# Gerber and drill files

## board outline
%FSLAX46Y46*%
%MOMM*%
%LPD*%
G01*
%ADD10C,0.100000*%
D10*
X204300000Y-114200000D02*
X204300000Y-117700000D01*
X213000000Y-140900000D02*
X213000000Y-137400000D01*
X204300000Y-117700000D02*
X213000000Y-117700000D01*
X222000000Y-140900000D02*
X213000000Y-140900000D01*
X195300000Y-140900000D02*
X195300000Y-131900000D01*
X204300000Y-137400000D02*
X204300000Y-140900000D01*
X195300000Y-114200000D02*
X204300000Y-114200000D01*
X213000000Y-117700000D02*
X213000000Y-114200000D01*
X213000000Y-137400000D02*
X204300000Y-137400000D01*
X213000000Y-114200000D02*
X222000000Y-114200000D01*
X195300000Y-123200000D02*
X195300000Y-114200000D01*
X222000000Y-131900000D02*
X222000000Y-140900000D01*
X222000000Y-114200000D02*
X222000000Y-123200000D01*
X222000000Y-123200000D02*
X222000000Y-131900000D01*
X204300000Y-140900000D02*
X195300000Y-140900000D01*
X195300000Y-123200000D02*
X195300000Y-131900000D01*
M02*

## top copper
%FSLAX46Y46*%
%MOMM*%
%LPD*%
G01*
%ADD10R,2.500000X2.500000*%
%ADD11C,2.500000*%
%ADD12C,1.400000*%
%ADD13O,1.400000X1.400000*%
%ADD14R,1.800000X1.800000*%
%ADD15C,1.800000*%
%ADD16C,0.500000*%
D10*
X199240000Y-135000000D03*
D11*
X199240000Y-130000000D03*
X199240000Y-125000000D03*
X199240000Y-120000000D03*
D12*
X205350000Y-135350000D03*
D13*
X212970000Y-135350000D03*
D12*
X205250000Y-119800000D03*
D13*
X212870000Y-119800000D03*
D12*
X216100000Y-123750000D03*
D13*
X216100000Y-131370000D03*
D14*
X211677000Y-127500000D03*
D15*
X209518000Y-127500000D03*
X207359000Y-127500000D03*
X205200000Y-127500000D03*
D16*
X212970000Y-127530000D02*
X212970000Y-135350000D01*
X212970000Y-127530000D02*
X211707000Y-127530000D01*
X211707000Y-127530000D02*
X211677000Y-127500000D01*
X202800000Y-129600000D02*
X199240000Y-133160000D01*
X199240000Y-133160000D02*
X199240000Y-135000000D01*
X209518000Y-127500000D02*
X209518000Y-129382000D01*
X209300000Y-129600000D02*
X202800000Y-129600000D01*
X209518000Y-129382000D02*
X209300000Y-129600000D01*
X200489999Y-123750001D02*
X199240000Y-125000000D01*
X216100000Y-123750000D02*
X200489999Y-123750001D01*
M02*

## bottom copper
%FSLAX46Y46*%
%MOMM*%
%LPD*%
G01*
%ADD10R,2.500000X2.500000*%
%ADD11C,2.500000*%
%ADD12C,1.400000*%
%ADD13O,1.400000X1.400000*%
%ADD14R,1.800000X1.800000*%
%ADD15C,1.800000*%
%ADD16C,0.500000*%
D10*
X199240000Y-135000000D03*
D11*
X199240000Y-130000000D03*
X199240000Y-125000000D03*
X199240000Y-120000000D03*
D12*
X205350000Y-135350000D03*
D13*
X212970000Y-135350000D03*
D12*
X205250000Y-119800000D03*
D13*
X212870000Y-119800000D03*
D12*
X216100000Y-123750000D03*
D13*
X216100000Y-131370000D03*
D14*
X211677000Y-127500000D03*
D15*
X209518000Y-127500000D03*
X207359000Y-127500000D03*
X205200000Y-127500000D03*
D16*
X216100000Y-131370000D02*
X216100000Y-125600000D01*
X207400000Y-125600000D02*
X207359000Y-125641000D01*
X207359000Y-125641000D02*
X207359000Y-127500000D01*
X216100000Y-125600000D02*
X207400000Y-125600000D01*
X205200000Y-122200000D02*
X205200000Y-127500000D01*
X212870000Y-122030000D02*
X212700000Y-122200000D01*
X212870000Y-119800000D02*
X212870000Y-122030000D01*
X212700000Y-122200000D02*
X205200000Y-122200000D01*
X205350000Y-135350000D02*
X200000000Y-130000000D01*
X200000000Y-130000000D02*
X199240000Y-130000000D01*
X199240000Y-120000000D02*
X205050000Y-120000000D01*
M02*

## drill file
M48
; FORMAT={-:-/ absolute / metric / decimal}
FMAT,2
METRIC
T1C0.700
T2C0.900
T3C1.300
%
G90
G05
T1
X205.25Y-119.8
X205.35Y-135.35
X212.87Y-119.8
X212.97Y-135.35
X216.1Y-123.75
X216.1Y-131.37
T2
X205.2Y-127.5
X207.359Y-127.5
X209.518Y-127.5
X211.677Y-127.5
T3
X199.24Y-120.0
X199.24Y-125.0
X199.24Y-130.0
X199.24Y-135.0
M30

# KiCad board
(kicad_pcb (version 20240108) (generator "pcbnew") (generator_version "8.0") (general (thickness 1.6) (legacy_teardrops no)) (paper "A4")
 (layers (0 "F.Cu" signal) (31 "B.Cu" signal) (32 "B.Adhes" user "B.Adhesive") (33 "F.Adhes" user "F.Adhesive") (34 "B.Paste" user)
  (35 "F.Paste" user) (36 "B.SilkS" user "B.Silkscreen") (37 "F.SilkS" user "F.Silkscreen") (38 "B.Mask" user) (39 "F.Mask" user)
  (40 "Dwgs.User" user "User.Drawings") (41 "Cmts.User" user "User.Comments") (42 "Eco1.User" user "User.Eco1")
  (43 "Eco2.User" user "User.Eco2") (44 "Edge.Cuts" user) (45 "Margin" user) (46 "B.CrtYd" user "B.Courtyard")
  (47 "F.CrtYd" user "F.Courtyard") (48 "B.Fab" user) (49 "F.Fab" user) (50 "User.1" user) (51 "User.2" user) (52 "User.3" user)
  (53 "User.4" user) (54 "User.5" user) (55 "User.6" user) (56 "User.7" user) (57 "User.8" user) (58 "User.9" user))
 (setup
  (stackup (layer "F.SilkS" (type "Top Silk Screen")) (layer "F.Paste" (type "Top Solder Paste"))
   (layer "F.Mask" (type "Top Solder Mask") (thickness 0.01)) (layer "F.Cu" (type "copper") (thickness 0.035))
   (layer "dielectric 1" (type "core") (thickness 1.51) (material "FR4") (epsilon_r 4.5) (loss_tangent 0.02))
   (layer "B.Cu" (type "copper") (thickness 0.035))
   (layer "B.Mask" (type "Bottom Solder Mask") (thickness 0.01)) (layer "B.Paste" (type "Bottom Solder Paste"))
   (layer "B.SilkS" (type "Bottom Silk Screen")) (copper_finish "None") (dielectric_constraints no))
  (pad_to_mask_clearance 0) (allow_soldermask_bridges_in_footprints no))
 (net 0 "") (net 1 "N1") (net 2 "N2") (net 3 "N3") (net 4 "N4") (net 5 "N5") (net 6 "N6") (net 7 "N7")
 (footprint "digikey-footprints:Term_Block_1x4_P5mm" (layer "F.Cu") (at 199.24 135 90)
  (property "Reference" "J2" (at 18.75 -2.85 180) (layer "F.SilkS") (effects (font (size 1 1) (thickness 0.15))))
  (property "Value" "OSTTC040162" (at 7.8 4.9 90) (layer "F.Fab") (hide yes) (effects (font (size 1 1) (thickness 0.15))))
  (pad "1" thru_hole rect (at 0 0 90) (size 2.5 2.5) (drill 1.3) (layers "*.Cu" "*.Mask") (remove_unused_layers no) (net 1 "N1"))
  (pad "2" thru_hole circle (at 5 0 90) (size 2.5 2.5) (drill 1.3) (layers "*.Cu" "*.Mask") (remove_unused_layers no) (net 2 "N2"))
  (pad "3" thru_hole circle (at 10 0 90) (size 2.5 2.5) (drill 1.3) (layers "*.Cu" "*.Mask") (remove_unused_layers no) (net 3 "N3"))
  (pad "4" thru_hole circle (at 15 0 90) (size 2.5 2.5) (drill 1.3) (layers "*.Cu" "*.Mask") (remove_unused_layers no) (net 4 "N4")))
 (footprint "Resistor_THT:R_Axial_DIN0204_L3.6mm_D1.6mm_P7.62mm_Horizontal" (layer "F.Cu") (at 205.35 135.35)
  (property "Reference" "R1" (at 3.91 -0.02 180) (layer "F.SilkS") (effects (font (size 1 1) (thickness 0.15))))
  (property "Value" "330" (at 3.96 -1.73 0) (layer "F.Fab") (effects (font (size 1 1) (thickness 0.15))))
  (pad "1" thru_hole circle (at 0 0) (size 1.4 1.4) (drill 0.7) (layers "*.Cu" "*.Mask") (remove_unused_layers no) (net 2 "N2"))
  (pad "2" thru_hole oval (at 7.62 0) (size 1.4 1.4) (drill 0.7) (layers "*.Cu" "*.Mask") (remove_unused_layers no) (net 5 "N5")))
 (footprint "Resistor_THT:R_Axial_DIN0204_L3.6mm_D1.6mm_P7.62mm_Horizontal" (layer "F.Cu") (at 205.25 119.8)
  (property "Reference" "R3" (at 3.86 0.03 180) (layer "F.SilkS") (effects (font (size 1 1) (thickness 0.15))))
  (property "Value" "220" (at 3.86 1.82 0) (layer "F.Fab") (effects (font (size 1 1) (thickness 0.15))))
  (pad "1" thru_hole circle (at 0 0) (size 1.4 1.4) (drill 0.7) (layers "*.Cu" "*.Mask") (remove_unused_layers no) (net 4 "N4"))
  (pad "2" thru_hole oval (at 7.62 0) (size 1.4 1.4) (drill 0.7) (layers "*.Cu" "*.Mask") (remove_unused_layers no) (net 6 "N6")))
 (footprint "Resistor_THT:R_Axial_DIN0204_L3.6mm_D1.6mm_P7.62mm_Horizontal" (layer "F.Cu") (at 216.1 123.75 -90)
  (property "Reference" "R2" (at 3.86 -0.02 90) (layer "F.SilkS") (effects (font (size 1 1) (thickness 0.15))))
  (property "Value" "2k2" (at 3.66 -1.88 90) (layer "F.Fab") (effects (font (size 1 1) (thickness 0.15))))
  (pad "1" thru_hole circle (at 0 0 270) (size 1.4 1.4) (drill 0.7) (layers "*.Cu" "*.Mask") (remove_unused_layers no) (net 3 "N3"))
  (pad "2" thru_hole oval (at 7.62 0 270) (size 1.4 1.4) (drill 0.7) (layers "*.Cu" "*.Mask") (remove_unused_layers no) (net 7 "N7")))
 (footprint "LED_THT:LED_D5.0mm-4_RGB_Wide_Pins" (layer "B.Cu") (at 211.677 127.5 180)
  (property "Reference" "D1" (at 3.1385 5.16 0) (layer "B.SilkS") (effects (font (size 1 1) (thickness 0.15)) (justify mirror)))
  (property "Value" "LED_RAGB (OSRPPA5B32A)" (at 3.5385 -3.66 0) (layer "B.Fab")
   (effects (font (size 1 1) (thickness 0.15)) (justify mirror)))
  (pad "1" thru_hole rect (at 0 0 180) (size 1.8 1.8) (drill 0.9) (layers "*.Cu" "*.Mask") (remove_unused_layers no) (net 5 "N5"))
  (pad "2" thru_hole circle (at 2.159 0 180) (size 1.8 1.8) (drill 0.9) (layers "*.Cu" "*.Mask") (remove_unused_layers no) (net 1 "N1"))
  (pad "3" thru_hole circle (at 4.318 0 180) (size 1.8 1.8) (drill 0.9) (layers "*.Cu" "*.Mask") (remove_unused_layers no) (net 7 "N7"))
  (pad "4" thru_hole circle (at 6.477 0 180) (size 1.8 1.8) (drill 0.9) (layers "*.Cu" "*.Mask") (remove_unused_layers no) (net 6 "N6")))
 (gr_line (start 204.3 114.2) (end 204.3 117.7) (stroke (width 0.1) (type solid)) (layer "Edge.Cuts"))
 (gr_line (start 213 140.9) (end 213 137.4) (stroke (width 0.1) (type solid)) (layer "Edge.Cuts"))
 (gr_line (start 204.3 117.7) (end 213 117.7) (stroke (width 0.1) (type solid)) (layer "Edge.Cuts"))
 (gr_line (start 222 140.9) (end 213 140.9) (stroke (width 0.1) (type solid)) (layer "Edge.Cuts"))
 (gr_line (start 195.3 140.9) (end 195.3 131.9) (stroke (width 0.1) (type solid)) (layer "Edge.Cuts"))
 (gr_line (start 204.3 137.4) (end 204.3 140.9) (stroke (width 0.1) (type solid)) (layer "Edge.Cuts"))
 (gr_line (start 195.3 114.2) (end 204.3 114.2) (stroke (width 0.1) (type solid)) (layer "Edge.Cuts"))
 (gr_line (start 213 117.7) (end 213 114.2) (stroke (width 0.1) (type solid)) (layer "Edge.Cuts"))
 (gr_line (start 213 137.4) (end 204.3 137.4) (stroke (width 0.1) (type solid)) (layer "Edge.Cuts"))
 (gr_line (start 213 114.2) (end 222 114.2) (stroke (width 0.1) (type solid)) (layer "Edge.Cuts"))
 (gr_line (start 195.3 123.2) (end 195.3 114.2) (stroke (width 0.1) (type solid)) (layer "Edge.Cuts"))
 (gr_line (start 222 131.9) (end 222 140.9) (stroke (width 0.1) (type solid)) (layer "Edge.Cuts"))
 (gr_line (start 222 114.2) (end 222 123.2) (stroke (width 0.1) (type solid)) (layer "Edge.Cuts"))
 (gr_line (start 222 123.2) (end 222 131.9) (stroke (width 0.1) (type solid)) (layer "Edge.Cuts"))
 (gr_line (start 204.3 140.9) (end 195.3 140.9) (stroke (width 0.1) (type solid)) (layer "Edge.Cuts"))
 (gr_line (start 195.3 123.2) (end 195.3 131.9) (stroke (width 0.1) (type solid)) (layer "Edge.Cuts"))
 (segment (start 212.97 127.53) (end 212.97 135.35) (width 0.5) (layer "F.Cu") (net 5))
 (segment (start 212.97 127.53) (end 211.707 127.53) (width 0.5) (layer "F.Cu") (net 5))
 (segment (start 211.707 127.53) (end 211.677 127.5) (width 0.5) (layer "F.Cu") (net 5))
 (segment (start 202.8 129.6) (end 199.24 133.16) (width 0.5) (layer "F.Cu") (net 1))
 (segment (start 199.24 133.16) (end 199.24 135) (width 0.5) (layer "F.Cu") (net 1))
 (segment (start 209.518 127.5) (end 209.518 129.382) (width 0.5) (layer "F.Cu") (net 1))
 (segment (start 209.3 129.6) (end 202.8 129.6) (width 0.5) (layer "F.Cu") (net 1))
 (segment (start 209.518 129.382) (end 209.3 129.6) (width 0.5) (layer "F.Cu") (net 1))
 (segment (start 216.1 131.37) (end 216.1 125.6) (width 0.5) (layer "B.Cu") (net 7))
 (segment (start 207.4 125.6) (end 207.359 125.641) (width 0.5) (layer "B.Cu") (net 7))
 (segment (start 207.359 125.641) (end 207.359 127.5) (width 0.5) (layer "B.Cu") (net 7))
 (segment (start 216.1 125.6) (end 207.4 125.6) (width 0.5) (layer "B.Cu") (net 7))
 (segment (start 205.2 122.2) (end 205.2 127.5) (width 0.5) (layer "B.Cu") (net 6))
 (segment (start 212.87 122.03) (end 212.7 122.2) (width 0.5) (layer "B.Cu") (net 6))
 (segment (start 212.87 119.8) (end 212.87 122.03) (width 0.5) (layer "B.Cu") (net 6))
 (segment (start 212.7 122.2) (end 205.2 122.2) (width 0.5) (layer "B.Cu") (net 6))
 (segment (start 205.35 135.35) (end 200 130) (width 0.5) (layer "B.Cu") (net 2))
 (segment (start 200 130) (end 199.24 130) (width 0.5) (layer "B.Cu") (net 2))
 (segment (start 200.489999 123.750001) (end 199.24 125) (width 0.5) (layer "F.Cu") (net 3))
 (segment (start 216.1 123.75) (end 200.489999 123.750001) (width 0.5) (layer "F.Cu") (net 3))
 (segment (start 199.24 120) (end 205.05 120) (width 0.5) (layer "B.Cu") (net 4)))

